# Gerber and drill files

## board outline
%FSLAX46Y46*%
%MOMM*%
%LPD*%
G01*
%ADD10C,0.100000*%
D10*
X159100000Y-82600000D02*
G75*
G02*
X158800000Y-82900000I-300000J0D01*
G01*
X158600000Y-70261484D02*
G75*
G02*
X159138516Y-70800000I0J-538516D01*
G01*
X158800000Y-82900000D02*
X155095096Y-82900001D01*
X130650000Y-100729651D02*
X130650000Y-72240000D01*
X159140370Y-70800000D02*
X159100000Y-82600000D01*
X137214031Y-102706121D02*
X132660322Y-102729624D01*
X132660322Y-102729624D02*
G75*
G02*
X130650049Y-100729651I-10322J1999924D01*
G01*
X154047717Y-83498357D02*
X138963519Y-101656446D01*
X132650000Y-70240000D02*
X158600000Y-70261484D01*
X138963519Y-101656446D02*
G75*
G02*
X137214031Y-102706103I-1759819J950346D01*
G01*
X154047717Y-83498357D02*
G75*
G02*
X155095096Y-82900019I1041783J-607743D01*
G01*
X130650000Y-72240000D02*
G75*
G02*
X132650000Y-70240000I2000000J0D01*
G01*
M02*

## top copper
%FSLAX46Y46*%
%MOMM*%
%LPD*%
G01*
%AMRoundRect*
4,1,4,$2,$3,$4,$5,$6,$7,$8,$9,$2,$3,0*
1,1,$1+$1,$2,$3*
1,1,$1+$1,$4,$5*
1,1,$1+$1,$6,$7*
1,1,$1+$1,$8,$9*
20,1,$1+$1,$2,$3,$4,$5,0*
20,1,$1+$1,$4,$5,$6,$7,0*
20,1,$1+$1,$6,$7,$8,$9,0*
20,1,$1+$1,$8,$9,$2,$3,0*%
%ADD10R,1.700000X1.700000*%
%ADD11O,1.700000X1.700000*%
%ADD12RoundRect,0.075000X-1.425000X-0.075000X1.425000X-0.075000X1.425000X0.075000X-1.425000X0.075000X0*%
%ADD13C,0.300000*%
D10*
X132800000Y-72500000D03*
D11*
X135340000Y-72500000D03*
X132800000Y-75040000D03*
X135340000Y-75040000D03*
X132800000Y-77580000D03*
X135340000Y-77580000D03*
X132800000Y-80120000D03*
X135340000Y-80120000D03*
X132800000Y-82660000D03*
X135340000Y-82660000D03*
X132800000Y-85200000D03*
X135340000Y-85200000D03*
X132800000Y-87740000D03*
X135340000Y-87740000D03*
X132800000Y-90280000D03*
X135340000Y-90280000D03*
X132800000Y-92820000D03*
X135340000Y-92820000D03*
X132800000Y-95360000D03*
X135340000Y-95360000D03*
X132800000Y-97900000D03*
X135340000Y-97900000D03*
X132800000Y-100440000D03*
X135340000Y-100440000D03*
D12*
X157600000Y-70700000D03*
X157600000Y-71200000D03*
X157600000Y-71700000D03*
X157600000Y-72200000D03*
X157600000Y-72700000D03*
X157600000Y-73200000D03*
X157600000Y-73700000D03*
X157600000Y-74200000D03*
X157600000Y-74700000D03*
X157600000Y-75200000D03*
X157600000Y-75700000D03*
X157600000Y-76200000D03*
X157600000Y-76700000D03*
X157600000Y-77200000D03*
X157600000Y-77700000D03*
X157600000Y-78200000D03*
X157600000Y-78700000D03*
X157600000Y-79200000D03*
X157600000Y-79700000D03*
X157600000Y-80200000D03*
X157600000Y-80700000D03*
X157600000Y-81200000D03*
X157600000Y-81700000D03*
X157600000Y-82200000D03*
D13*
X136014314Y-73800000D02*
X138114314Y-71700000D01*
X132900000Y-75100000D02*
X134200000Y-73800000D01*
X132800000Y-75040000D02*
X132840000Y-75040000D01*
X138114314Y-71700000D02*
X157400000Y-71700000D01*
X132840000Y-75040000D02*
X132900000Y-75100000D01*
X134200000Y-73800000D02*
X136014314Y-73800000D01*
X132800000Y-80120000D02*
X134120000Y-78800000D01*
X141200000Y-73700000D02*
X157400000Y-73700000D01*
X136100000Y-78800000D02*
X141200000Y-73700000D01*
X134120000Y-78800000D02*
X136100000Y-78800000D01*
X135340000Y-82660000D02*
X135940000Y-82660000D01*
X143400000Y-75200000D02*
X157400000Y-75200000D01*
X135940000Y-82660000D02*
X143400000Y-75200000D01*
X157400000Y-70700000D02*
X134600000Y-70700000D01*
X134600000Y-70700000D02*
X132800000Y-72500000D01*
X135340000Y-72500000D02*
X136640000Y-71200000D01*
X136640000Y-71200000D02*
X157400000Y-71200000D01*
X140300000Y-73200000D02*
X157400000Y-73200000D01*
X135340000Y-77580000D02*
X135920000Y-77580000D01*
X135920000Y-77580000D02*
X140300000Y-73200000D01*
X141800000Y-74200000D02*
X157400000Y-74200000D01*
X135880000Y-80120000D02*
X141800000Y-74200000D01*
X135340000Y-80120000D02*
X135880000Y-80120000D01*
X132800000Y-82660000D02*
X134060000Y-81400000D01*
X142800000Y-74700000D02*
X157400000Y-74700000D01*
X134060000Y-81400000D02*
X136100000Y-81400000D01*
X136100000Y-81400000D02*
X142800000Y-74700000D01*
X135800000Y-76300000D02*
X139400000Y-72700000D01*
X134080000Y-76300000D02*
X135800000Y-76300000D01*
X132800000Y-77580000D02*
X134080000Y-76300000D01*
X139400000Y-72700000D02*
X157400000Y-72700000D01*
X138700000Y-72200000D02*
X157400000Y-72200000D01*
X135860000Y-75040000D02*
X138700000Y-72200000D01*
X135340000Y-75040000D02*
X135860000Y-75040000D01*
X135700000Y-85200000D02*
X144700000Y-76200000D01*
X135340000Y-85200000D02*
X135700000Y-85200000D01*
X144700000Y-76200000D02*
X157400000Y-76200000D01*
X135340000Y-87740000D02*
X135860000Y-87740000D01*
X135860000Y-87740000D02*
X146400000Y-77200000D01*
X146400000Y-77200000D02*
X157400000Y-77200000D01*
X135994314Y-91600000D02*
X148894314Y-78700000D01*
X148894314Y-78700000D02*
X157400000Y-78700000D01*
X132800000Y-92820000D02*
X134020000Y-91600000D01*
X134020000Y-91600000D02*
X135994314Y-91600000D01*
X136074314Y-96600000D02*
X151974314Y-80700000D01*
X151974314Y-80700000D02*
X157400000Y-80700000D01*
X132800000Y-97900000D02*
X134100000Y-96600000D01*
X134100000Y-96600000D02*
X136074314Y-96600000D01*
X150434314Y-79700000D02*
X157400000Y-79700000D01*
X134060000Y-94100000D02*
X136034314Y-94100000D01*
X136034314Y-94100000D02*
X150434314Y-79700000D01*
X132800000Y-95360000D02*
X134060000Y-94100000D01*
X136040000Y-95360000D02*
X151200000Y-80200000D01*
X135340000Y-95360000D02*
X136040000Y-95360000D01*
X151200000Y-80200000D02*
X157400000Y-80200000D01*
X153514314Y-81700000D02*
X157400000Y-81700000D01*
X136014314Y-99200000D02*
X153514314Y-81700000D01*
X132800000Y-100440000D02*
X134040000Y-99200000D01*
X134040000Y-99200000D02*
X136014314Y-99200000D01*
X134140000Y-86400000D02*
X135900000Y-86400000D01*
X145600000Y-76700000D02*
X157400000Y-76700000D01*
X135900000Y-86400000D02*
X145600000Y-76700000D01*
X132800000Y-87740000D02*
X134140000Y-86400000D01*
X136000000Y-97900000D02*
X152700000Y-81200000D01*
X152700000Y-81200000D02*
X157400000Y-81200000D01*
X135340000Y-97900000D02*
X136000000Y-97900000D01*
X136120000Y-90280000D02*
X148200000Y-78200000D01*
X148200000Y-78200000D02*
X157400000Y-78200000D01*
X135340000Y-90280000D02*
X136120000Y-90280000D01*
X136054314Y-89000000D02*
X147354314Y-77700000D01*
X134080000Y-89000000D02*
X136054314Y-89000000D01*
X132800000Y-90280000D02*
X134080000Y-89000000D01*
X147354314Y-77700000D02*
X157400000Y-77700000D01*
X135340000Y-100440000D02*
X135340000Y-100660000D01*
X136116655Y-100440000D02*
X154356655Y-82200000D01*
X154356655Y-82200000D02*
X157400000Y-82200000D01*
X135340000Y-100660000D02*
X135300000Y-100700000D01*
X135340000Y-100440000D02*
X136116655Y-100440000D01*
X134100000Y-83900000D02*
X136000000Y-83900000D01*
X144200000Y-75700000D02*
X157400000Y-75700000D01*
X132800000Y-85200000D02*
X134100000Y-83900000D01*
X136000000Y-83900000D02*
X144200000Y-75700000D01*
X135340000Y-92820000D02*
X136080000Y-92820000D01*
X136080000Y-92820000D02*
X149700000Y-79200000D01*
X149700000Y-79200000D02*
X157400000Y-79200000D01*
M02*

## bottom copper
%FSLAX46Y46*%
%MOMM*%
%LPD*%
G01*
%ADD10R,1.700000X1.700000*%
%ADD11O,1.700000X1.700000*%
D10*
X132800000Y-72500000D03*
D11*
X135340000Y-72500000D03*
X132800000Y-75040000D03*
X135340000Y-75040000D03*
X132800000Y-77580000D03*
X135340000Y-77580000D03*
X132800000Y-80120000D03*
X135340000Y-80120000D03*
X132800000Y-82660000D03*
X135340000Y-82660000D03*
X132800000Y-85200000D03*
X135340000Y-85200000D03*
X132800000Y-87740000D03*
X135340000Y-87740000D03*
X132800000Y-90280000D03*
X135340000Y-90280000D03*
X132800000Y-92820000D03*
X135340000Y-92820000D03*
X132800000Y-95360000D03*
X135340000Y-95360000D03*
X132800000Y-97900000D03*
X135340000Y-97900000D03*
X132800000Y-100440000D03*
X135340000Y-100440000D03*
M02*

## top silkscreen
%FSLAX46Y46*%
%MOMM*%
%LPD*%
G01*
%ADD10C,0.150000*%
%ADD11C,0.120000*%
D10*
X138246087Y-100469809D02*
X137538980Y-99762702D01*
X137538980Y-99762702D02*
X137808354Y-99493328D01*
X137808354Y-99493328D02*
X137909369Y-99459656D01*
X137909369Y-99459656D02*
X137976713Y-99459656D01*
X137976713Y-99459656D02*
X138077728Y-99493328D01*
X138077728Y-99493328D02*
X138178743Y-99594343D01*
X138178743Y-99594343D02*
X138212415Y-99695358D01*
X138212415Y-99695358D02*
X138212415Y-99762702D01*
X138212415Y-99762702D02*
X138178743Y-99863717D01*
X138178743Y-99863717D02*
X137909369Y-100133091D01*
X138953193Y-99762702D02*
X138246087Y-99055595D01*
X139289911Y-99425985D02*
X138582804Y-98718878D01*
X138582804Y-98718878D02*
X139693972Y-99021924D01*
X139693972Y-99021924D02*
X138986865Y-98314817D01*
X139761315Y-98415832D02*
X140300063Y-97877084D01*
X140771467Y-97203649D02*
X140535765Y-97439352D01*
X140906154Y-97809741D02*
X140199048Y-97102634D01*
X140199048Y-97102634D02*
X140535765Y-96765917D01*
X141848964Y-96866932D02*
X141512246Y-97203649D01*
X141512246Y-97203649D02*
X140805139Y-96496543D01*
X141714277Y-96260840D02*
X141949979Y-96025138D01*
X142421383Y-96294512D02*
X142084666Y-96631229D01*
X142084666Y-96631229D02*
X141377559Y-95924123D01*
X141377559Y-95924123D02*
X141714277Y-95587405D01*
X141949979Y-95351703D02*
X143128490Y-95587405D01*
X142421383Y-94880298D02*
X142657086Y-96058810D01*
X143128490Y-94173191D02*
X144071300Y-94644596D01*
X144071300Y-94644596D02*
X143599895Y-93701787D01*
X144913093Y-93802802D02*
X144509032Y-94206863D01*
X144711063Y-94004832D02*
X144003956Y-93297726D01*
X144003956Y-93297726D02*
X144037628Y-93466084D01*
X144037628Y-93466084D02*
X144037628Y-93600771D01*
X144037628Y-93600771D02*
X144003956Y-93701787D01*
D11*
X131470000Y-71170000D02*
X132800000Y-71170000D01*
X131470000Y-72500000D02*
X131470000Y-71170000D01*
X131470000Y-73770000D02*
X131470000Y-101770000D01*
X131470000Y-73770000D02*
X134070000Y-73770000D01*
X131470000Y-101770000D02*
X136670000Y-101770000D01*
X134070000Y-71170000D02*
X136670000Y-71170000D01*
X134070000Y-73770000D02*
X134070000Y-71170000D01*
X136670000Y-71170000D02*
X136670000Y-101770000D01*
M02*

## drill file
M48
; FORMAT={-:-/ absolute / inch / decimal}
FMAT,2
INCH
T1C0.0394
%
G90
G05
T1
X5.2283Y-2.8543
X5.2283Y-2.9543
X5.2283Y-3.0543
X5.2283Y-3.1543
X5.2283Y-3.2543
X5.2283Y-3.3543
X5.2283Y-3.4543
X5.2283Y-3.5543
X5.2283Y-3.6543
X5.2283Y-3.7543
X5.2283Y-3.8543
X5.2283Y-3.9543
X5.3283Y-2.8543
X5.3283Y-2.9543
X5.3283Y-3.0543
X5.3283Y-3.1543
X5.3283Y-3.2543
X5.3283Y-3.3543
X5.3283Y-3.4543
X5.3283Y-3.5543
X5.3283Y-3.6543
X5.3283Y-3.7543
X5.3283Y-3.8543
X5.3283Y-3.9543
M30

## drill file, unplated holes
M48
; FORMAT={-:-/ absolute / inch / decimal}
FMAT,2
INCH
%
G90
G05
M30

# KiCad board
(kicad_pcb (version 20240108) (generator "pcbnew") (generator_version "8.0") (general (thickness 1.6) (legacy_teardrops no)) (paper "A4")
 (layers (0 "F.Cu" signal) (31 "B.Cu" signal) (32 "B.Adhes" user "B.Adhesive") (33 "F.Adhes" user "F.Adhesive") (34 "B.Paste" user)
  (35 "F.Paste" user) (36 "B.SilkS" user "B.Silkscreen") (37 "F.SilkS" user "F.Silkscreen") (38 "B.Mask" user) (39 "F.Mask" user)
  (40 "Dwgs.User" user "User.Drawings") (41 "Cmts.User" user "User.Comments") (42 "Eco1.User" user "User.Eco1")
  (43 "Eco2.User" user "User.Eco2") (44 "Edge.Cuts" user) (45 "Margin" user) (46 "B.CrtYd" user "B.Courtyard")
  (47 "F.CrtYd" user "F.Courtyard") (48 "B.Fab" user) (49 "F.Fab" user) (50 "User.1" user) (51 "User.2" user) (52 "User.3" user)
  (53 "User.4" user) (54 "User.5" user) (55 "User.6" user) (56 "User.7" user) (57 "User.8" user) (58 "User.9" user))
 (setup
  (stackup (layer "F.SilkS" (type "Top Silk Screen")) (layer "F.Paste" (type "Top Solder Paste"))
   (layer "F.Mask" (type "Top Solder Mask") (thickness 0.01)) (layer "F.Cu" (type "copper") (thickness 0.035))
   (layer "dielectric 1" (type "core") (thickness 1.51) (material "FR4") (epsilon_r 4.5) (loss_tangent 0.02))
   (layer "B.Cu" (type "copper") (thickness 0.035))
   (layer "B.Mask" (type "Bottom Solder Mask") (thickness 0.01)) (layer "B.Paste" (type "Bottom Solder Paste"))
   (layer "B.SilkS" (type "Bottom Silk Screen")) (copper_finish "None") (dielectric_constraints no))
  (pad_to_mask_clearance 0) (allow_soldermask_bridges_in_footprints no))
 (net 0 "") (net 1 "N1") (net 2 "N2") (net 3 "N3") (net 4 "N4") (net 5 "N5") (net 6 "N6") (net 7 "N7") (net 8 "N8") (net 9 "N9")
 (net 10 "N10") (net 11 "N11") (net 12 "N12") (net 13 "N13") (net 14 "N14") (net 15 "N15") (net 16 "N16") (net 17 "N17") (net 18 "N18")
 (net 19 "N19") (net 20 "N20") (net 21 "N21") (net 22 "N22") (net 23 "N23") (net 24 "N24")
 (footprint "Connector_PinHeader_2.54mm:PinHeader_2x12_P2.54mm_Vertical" (layer "F.Cu") (at 132.8 72.5)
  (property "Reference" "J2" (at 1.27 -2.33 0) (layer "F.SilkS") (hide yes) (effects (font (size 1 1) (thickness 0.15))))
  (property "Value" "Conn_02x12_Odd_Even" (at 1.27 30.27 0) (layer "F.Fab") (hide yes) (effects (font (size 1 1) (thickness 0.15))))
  (fp_line (start -1.33 -1.33) (end 0 -1.33) (stroke (width 0.12) (type solid)) (layer "F.SilkS"))
  (fp_line (start -1.33 0) (end -1.33 -1.33) (stroke (width 0.12) (type solid)) (layer "F.SilkS"))
  (fp_line (start -1.33 1.27) (end -1.33 29.27) (stroke (width 0.12) (type solid)) (layer "F.SilkS"))
  (fp_line (start -1.33 1.27) (end 1.27 1.27) (stroke (width 0.12) (type solid)) (layer "F.SilkS"))
  (fp_line (start -1.33 29.27) (end 3.87 29.27) (stroke (width 0.12) (type solid)) (layer "F.SilkS"))
  (fp_line (start 1.27 -1.33) (end 3.87 -1.33) (stroke (width 0.12) (type solid)) (layer "F.SilkS"))
  (fp_line (start 1.27 1.27) (end 1.27 -1.33) (stroke (width 0.12) (type solid)) (layer "F.SilkS"))
  (fp_line (start 3.87 -1.33) (end 3.87 29.27) (stroke (width 0.12) (type solid)) (layer "F.SilkS"))
  (pad "1" thru_hole rect (at 0 0) (size 1.7 1.7) (drill 1) (layers "*.Cu" "*.Mask") (remove_unused_layers no) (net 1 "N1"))
  (pad "2" thru_hole oval (at 2.54 0) (size 1.7 1.7) (drill 1) (layers "*.Cu" "*.Mask") (remove_unused_layers no) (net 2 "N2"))
  (pad "3" thru_hole oval (at 0 2.54) (size 1.7 1.7) (drill 1) (layers "*.Cu" "*.Mask") (remove_unused_layers no) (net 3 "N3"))
  (pad "4" thru_hole oval (at 2.54 2.54) (size 1.7 1.7) (drill 1) (layers "*.Cu" "*.Mask") (remove_unused_layers no) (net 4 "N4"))
  (pad "5" thru_hole oval (at 0 5.08) (size 1.7 1.7) (drill 1) (layers "*.Cu" "*.Mask") (remove_unused_layers no) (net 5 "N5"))
  (pad "6" thru_hole oval (at 2.54 5.08) (size 1.7 1.7) (drill 1) (layers "*.Cu" "*.Mask") (remove_unused_layers no) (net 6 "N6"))
  (pad "7" thru_hole oval (at 0 7.62) (size 1.7 1.7) (drill 1) (layers "*.Cu" "*.Mask") (remove_unused_layers no) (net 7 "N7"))
  (pad "8" thru_hole oval (at 2.54 7.62) (size 1.7 1.7) (drill 1) (layers "*.Cu" "*.Mask") (remove_unused_layers no) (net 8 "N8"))
  (pad "9" thru_hole oval (at 0 10.16) (size 1.7 1.7) (drill 1) (layers "*.Cu" "*.Mask") (remove_unused_layers no) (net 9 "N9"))
  (pad "10" thru_hole oval (at 2.54 10.16) (size 1.7 1.7) (drill 1) (layers "*.Cu" "*.Mask") (remove_unused_layers no) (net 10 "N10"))
  (pad "11" thru_hole oval (at 0 12.7) (size 1.7 1.7) (drill 1) (layers "*.Cu" "*.Mask") (remove_unused_layers no) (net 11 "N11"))
  (pad "12" thru_hole oval (at 2.54 12.7) (size 1.7 1.7) (drill 1) (layers "*.Cu" "*.Mask") (remove_unused_layers no) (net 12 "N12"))
  (pad "13" thru_hole oval (at 0 15.24) (size 1.7 1.7) (drill 1) (layers "*.Cu" "*.Mask") (remove_unused_layers no) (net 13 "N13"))
  (pad "14" thru_hole oval (at 2.54 15.24) (size 1.7 1.7) (drill 1) (layers "*.Cu" "*.Mask") (remove_unused_layers no) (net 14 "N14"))
  (pad "15" thru_hole oval (at 0 17.78) (size 1.7 1.7) (drill 1) (layers "*.Cu" "*.Mask") (remove_unused_layers no) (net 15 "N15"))
  (pad "16" thru_hole oval (at 2.54 17.78) (size 1.7 1.7) (drill 1) (layers "*.Cu" "*.Mask") (remove_unused_layers no) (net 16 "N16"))
  (pad "17" thru_hole oval (at 0 20.32) (size 1.7 1.7) (drill 1) (layers "*.Cu" "*.Mask") (remove_unused_layers no) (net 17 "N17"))
  (pad "18" thru_hole oval (at 2.54 20.32) (size 1.7 1.7) (drill 1) (layers "*.Cu" "*.Mask") (remove_unused_layers no) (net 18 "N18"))
  (pad "19" thru_hole oval (at 0 22.86) (size 1.7 1.7) (drill 1) (layers "*.Cu" "*.Mask") (remove_unused_layers no) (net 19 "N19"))
  (pad "20" thru_hole oval (at 2.54 22.86) (size 1.7 1.7) (drill 1) (layers "*.Cu" "*.Mask") (remove_unused_layers no) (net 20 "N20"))
  (pad "21" thru_hole oval (at 0 25.4) (size 1.7 1.7) (drill 1) (layers "*.Cu" "*.Mask") (remove_unused_layers no) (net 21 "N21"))
  (pad "22" thru_hole oval (at 2.54 25.4) (size 1.7 1.7) (drill 1) (layers "*.Cu" "*.Mask") (remove_unused_layers no) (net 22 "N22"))
  (pad "23" thru_hole oval (at 0 27.94) (size 1.7 1.7) (drill 1) (layers "*.Cu" "*.Mask") (remove_unused_layers no) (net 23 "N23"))
  (pad "24" thru_hole oval (at 2.54 27.94) (size 1.7 1.7) (drill 1) (layers "*.Cu" "*.Mask") (remove_unused_layers no) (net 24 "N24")))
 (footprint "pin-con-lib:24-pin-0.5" (layer "F.Cu") (at 157.6 70.7)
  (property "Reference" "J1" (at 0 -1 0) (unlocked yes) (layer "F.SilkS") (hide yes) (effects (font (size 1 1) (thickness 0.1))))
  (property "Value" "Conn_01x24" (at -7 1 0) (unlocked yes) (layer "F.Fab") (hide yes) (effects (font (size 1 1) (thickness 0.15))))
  (pad "1" smd roundrect (at 0 0) (size 3 0.3) (layers "F.Cu" "F.Paste" "F.Mask") (roundrect_rratio 0.25) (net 1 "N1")
   (thermal_bridge_angle 45))
  (pad "2" smd roundrect (at 0 0.5) (size 3 0.3) (layers "F.Cu" "F.Paste" "F.Mask") (roundrect_rratio 0.25) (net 2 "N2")
   (thermal_bridge_angle 45))
  (pad "3" smd roundrect (at 0 1) (size 3 0.3) (layers "F.Cu" "F.Paste" "F.Mask") (roundrect_rratio 0.25) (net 3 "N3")
   (thermal_bridge_angle 45))
  (pad "4" smd roundrect (at 0 1.5) (size 3 0.3) (layers "F.Cu" "F.Paste" "F.Mask") (roundrect_rratio 0.25) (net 4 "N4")
   (thermal_bridge_angle 45))
  (pad "5" smd roundrect (at 0 2) (size 3 0.3) (layers "F.Cu" "F.Paste" "F.Mask") (roundrect_rratio 0.25) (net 5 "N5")
   (thermal_bridge_angle 45))
  (pad "6" smd roundrect (at 0 2.5) (size 3 0.3) (layers "F.Cu" "F.Paste" "F.Mask") (roundrect_rratio 0.25) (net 6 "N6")
   (thermal_bridge_angle 45))
  (pad "7" smd roundrect (at 0 3) (size 3 0.3) (layers "F.Cu" "F.Paste" "F.Mask") (roundrect_rratio 0.25) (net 7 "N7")
   (thermal_bridge_angle 45))
  (pad "8" smd roundrect (at 0 3.5) (size 3 0.3) (layers "F.Cu" "F.Paste" "F.Mask") (roundrect_rratio 0.25) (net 8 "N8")
   (thermal_bridge_angle 45))
  (pad "9" smd roundrect (at 0 4) (size 3 0.3) (layers "F.Cu" "F.Paste" "F.Mask") (roundrect_rratio 0.25) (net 9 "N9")
   (thermal_bridge_angle 45))
  (pad "10" smd roundrect (at 0 4.5) (size 3 0.3) (layers "F.Cu" "F.Paste" "F.Mask") (roundrect_rratio 0.25) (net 10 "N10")
   (thermal_bridge_angle 45))
  (pad "11" smd roundrect (at 0 5) (size 3 0.3) (layers "F.Cu" "F.Paste" "F.Mask") (roundrect_rratio 0.25) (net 11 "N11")
   (thermal_bridge_angle 45))
  (pad "12" smd roundrect (at 0 5.5) (size 3 0.3) (layers "F.Cu" "F.Paste" "F.Mask") (roundrect_rratio 0.25) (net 12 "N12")
   (thermal_bridge_angle 45))
  (pad "13" smd roundrect (at 0 6) (size 3 0.3) (layers "F.Cu" "F.Paste" "F.Mask") (roundrect_rratio 0.25) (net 13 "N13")
   (thermal_bridge_angle 45))
  (pad "14" smd roundrect (at 0 6.5) (size 3 0.3) (layers "F.Cu" "F.Paste" "F.Mask") (roundrect_rratio 0.25) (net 14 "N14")
   (thermal_bridge_angle 45))
  (pad "15" smd roundrect (at 0 7) (size 3 0.3) (layers "F.Cu" "F.Paste" "F.Mask") (roundrect_rratio 0.25) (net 15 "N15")
   (thermal_bridge_angle 45))
  (pad "16" smd roundrect (at 0 7.5) (size 3 0.3) (layers "F.Cu" "F.Paste" "F.Mask") (roundrect_rratio 0.25) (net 16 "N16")
   (thermal_bridge_angle 45))
  (pad "17" smd roundrect (at 0 8) (size 3 0.3) (layers "F.Cu" "F.Paste" "F.Mask") (roundrect_rratio 0.25) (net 17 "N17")
   (thermal_bridge_angle 45))
  (pad "18" smd roundrect (at 0 8.5) (size 3 0.3) (layers "F.Cu" "F.Paste" "F.Mask") (roundrect_rratio 0.25) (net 18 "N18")
   (thermal_bridge_angle 45))
  (pad "19" smd roundrect (at 0 9) (size 3 0.3) (layers "F.Cu" "F.Paste" "F.Mask") (roundrect_rratio 0.25) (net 19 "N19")
   (thermal_bridge_angle 45))
  (pad "20" smd roundrect (at 0 9.5) (size 3 0.3) (layers "F.Cu" "F.Paste" "F.Mask") (roundrect_rratio 0.25) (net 20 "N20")
   (thermal_bridge_angle 45))
  (pad "21" smd roundrect (at 0 10) (size 3 0.3) (layers "F.Cu" "F.Paste" "F.Mask") (roundrect_rratio 0.25) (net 21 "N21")
   (thermal_bridge_angle 45))
  (pad "22" smd roundrect (at 0 10.5) (size 3 0.3) (layers "F.Cu" "F.Paste" "F.Mask") (roundrect_rratio 0.25) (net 22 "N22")
   (thermal_bridge_angle 45))
  (pad "23" smd roundrect (at 0 11) (size 3 0.3) (layers "F.Cu" "F.Paste" "F.Mask") (roundrect_rratio 0.25) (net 23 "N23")
   (thermal_bridge_angle 45))
  (pad "24" smd roundrect (at 0 11.5) (size 3 0.3) (layers "F.Cu" "F.Paste" "F.Mask") (roundrect_rratio 0.25) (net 24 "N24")
   (thermal_bridge_angle 45)))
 (gr_arc (start 159.1 82.6) (mid 159.012132 82.812132) (end 158.8 82.9) (stroke (width 0.1) (type default)) (layer "Edge.Cuts"))
 (gr_arc (start 158.6 70.261484) (mid 158.980788 70.419212) (end 159.138516 70.8) (stroke (width 0.1) (type default)) (layer "Edge.Cuts"))
 (gr_line (start 158.8 82.9) (end 155.095096 82.900001) (stroke (width 0.1) (type default)) (layer "Edge.Cuts"))
 (gr_line (start 130.65 100.729651) (end 130.65 72.24) (stroke (width 0.1) (type default)) (layer "Edge.Cuts"))
 (gr_line (start 159.14037 70.8) (end 159.1 82.6) (stroke (width 0.1) (type default)) (layer "Edge.Cuts"))
 (gr_line (start 137.214031 102.706121) (end 132.660322 102.729624) (stroke (width 0.1) (type default)) (layer "Edge.Cuts"))
 (gr_arc (start 132.660322 102.729624) (mid 131.239441 102.147509) (end 130.65 100.729651) (stroke (width 0.1) (type default))
  (layer "Edge.Cuts"))
 (gr_line (start 154.047717 83.498357) (end 138.963519 101.656446) (stroke (width 0.1) (type default)) (layer "Edge.Cuts"))
 (gr_line (start 132.65 70.24) (end 158.6 70.261484) (stroke (width 0.1) (type default)) (layer "Edge.Cuts"))
 (gr_arc (start 138.963519 101.656446) (mid 138.232681 102.421127) (end 137.214031 102.706121) (stroke (width 0.1) (type default))
  (layer "Edge.Cuts"))
 (gr_arc (start 154.047717 83.498357) (mid 154.491229 83.058834) (end 155.095096 82.900001) (stroke (width 0.1) (type default))
  (layer "Edge.Cuts"))
 (gr_arc (start 130.65 72.24) (mid 131.235786 70.825786) (end 132.65 70.24) (stroke (width 0.1) (type default)) (layer "Edge.Cuts"))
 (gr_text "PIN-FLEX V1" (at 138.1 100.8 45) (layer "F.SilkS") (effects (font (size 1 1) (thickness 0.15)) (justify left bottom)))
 (segment (start 136.014314 73.8) (end 138.114314 71.7) (width 0.3) (layer "F.Cu") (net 3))
 (segment (start 132.9 75.1) (end 134.2 73.8) (width 0.3) (layer "F.Cu") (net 3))
 (segment (start 132.8 75.04) (end 132.84 75.04) (width 0.3) (layer "F.Cu") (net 3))
 (segment (start 138.114314 71.7) (end 157.4 71.7) (width 0.3) (layer "F.Cu") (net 3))
 (segment (start 132.84 75.04) (end 132.9 75.1) (width 0.3) (layer "F.Cu") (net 3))
 (segment (start 134.2 73.8) (end 136.014314 73.8) (width 0.3) (layer "F.Cu") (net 3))
 (segment (start 132.8 80.12) (end 134.12 78.8) (width 0.3) (layer "F.Cu") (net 7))
 (segment (start 141.2 73.7) (end 157.4 73.7) (width 0.3) (layer "F.Cu") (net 7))
 (segment (start 136.1 78.8) (end 141.2 73.7) (width 0.3) (layer "F.Cu") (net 7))
 (segment (start 134.12 78.8) (end 136.1 78.8) (width 0.3) (layer "F.Cu") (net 7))
 (segment (start 135.34 82.66) (end 135.94 82.66) (width 0.3) (layer "F.Cu") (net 10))
 (segment (start 143.4 75.2) (end 157.4 75.2) (width 0.3) (layer "F.Cu") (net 10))
 (segment (start 135.94 82.66) (end 143.4 75.2) (width 0.3) (layer "F.Cu") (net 10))
 (segment (start 157.4 70.7) (end 134.6 70.7) (width 0.3) (layer "F.Cu") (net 1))
 (segment (start 134.6 70.7) (end 132.8 72.5) (width 0.3) (layer "F.Cu") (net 1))
 (segment (start 135.34 72.5) (end 136.64 71.2) (width 0.3) (layer "F.Cu") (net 2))
 (segment (start 136.64 71.2) (end 157.4 71.2) (width 0.3) (layer "F.Cu") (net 2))
 (segment (start 140.3 73.2) (end 157.4 73.2) (width 0.3) (layer "F.Cu") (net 6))
 (segment (start 135.34 77.58) (end 135.92 77.58) (width 0.3) (layer "F.Cu") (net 6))
 (segment (start 135.92 77.58) (end 140.3 73.2) (width 0.3) (layer "F.Cu") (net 6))
 (segment (start 141.8 74.2) (end 157.4 74.2) (width 0.3) (layer "F.Cu") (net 8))
 (segment (start 135.88 80.12) (end 141.8 74.2) (width 0.3) (layer "F.Cu") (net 8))
 (segment (start 135.34 80.12) (end 135.88 80.12) (width 0.3) (layer "F.Cu") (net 8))
 (segment (start 132.8 82.66) (end 134.06 81.4) (width 0.3) (layer "F.Cu") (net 9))
 (segment (start 142.8 74.7) (end 157.4 74.7) (width 0.3) (layer "F.Cu") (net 9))
 (segment (start 134.06 81.4) (end 136.1 81.4) (width 0.3) (layer "F.Cu") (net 9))
 (segment (start 136.1 81.4) (end 142.8 74.7) (width 0.3) (layer "F.Cu") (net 9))
 (segment (start 135.8 76.3) (end 139.4 72.7) (width 0.3) (layer "F.Cu") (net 5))
 (segment (start 134.08 76.3) (end 135.8 76.3) (width 0.3) (layer "F.Cu") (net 5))
 (segment (start 132.8 77.58) (end 134.08 76.3) (width 0.3) (layer "F.Cu") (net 5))
 (segment (start 139.4 72.7) (end 157.4 72.7) (width 0.3) (layer "F.Cu") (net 5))
 (segment (start 138.7 72.2) (end 157.4 72.2) (width 0.3) (layer "F.Cu") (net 4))
 (segment (start 135.86 75.04) (end 138.7 72.2) (width 0.3) (layer "F.Cu") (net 4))
 (segment (start 135.34 75.04) (end 135.86 75.04) (width 0.3) (layer "F.Cu") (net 4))
 (segment (start 135.7 85.2) (end 144.7 76.2) (width 0.3) (layer "F.Cu") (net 12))
 (segment (start 135.34 85.2) (end 135.7 85.2) (width 0.3) (layer "F.Cu") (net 12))
 (segment (start 144.7 76.2) (end 157.4 76.2) (width 0.3) (layer "F.Cu") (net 12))
 (segment (start 135.34 87.74) (end 135.86 87.74) (width 0.3) (layer "F.Cu") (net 14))
 (segment (start 135.86 87.74) (end 146.4 77.2) (width 0.3) (layer "F.Cu") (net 14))
 (segment (start 146.4 77.2) (end 157.4 77.2) (width 0.3) (layer "F.Cu") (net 14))
 (segment (start 135.994314 91.6) (end 148.894314 78.7) (width 0.3) (layer "F.Cu") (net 17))
 (segment (start 148.894314 78.7) (end 157.4 78.7) (width 0.3) (layer "F.Cu") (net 17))
 (segment (start 132.8 92.82) (end 134.02 91.6) (width 0.3) (layer "F.Cu") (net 17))
 (segment (start 134.02 91.6) (end 135.994314 91.6) (width 0.3) (layer "F.Cu") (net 17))
 (segment (start 136.074314 96.6) (end 151.974314 80.7) (width 0.3) (layer "F.Cu") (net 21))
 (segment (start 151.974314 80.7) (end 157.4 80.7) (width 0.3) (layer "F.Cu") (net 21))
 (segment (start 132.8 97.9) (end 134.1 96.6) (width 0.3) (layer "F.Cu") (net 21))
 (segment (start 134.1 96.6) (end 136.074314 96.6) (width 0.3) (layer "F.Cu") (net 21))
 (segment (start 150.434314 79.7) (end 157.4 79.7) (width 0.3) (layer "F.Cu") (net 19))
 (segment (start 134.06 94.1) (end 136.034314 94.1) (width 0.3) (layer "F.Cu") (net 19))
 (segment (start 136.034314 94.1) (end 150.434314 79.7) (width 0.3) (layer "F.Cu") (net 19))
 (segment (start 132.8 95.36) (end 134.06 94.1) (width 0.3) (layer "F.Cu") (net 19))
 (segment (start 136.04 95.36) (end 151.2 80.2) (width 0.3) (layer "F.Cu") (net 20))
 (segment (start 135.34 95.36) (end 136.04 95.36) (width 0.3) (layer "F.Cu") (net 20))
 (segment (start 151.2 80.2) (end 157.4 80.2) (width 0.3) (layer "F.Cu") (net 20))
 (segment (start 153.514314 81.7) (end 157.4 81.7) (width 0.3) (layer "F.Cu") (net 23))
 (segment (start 136.014314 99.2) (end 153.514314 81.7) (width 0.3) (layer "F.Cu") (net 23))
 (segment (start 132.8 100.44) (end 134.04 99.2) (width 0.3) (layer "F.Cu") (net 23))
 (segment (start 134.04 99.2) (end 136.014314 99.2) (width 0.3) (layer "F.Cu") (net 23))
 (segment (start 134.14 86.4) (end 135.9 86.4) (width 0.3) (layer "F.Cu") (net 13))
 (segment (start 145.6 76.7) (end 157.4 76.7) (width 0.3) (layer "F.Cu") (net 13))
 (segment (start 135.9 86.4) (end 145.6 76.7) (width 0.3) (layer "F.Cu") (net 13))
 (segment (start 132.8 87.74) (end 134.14 86.4) (width 0.3) (layer "F.Cu") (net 13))
 (segment (start 136 97.9) (end 152.7 81.2) (width 0.3) (layer "F.Cu") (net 22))
 (segment (start 152.7 81.2) (end 157.4 81.2) (width 0.3) (layer "F.Cu") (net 22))
 (segment (start 135.34 97.9) (end 136 97.9) (width 0.3) (layer "F.Cu") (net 22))
 (segment (start 136.12 90.28) (end 148.2 78.2) (width 0.3) (layer "F.Cu") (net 16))
 (segment (start 148.2 78.2) (end 157.4 78.2) (width 0.3) (layer "F.Cu") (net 16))
 (segment (start 135.34 90.28) (end 136.12 90.28) (width 0.3) (layer "F.Cu") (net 16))
 (segment (start 136.054314 89) (end 147.354314 77.7) (width 0.3) (layer "F.Cu") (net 15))
 (segment (start 134.08 89) (end 136.054314 89) (width 0.3) (layer "F.Cu") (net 15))
 (segment (start 132.8 90.28) (end 134.08 89) (width 0.3) (layer "F.Cu") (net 15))
 (segment (start 147.354314 77.7) (end 157.4 77.7) (width 0.3) (layer "F.Cu") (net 15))
 (segment (start 135.34 100.44) (end 135.34 100.66) (width 0.3) (layer "F.Cu") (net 24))
 (segment (start 136.116655 100.44) (end 154.356655 82.2) (width 0.3) (layer "F.Cu") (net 24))
 (segment (start 154.356655 82.2) (end 157.4 82.2) (width 0.3) (layer "F.Cu") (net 24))
 (segment (start 135.34 100.66) (end 135.3 100.7) (width 0.3) (layer "F.Cu") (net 24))
 (segment (start 135.34 100.44) (end 136.116655 100.44) (width 0.3) (layer "F.Cu") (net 24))
 (segment (start 134.1 83.9) (end 136 83.9) (width 0.3) (layer "F.Cu") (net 11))
 (segment (start 144.2 75.7) (end 157.4 75.7) (width 0.3) (layer "F.Cu") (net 11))
 (segment (start 132.8 85.2) (end 134.1 83.9) (width 0.3) (layer "F.Cu") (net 11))
 (segment (start 136 83.9) (end 144.2 75.7) (width 0.3) (layer "F.Cu") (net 11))
 (segment (start 135.34 92.82) (end 136.08 92.82) (width 0.3) (layer "F.Cu") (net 18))
 (segment (start 136.08 92.82) (end 149.7 79.2) (width 0.3) (layer "F.Cu") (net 18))
 (segment (start 149.7 79.2) (end 157.4 79.2) (width 0.3) (layer "F.Cu") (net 18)))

